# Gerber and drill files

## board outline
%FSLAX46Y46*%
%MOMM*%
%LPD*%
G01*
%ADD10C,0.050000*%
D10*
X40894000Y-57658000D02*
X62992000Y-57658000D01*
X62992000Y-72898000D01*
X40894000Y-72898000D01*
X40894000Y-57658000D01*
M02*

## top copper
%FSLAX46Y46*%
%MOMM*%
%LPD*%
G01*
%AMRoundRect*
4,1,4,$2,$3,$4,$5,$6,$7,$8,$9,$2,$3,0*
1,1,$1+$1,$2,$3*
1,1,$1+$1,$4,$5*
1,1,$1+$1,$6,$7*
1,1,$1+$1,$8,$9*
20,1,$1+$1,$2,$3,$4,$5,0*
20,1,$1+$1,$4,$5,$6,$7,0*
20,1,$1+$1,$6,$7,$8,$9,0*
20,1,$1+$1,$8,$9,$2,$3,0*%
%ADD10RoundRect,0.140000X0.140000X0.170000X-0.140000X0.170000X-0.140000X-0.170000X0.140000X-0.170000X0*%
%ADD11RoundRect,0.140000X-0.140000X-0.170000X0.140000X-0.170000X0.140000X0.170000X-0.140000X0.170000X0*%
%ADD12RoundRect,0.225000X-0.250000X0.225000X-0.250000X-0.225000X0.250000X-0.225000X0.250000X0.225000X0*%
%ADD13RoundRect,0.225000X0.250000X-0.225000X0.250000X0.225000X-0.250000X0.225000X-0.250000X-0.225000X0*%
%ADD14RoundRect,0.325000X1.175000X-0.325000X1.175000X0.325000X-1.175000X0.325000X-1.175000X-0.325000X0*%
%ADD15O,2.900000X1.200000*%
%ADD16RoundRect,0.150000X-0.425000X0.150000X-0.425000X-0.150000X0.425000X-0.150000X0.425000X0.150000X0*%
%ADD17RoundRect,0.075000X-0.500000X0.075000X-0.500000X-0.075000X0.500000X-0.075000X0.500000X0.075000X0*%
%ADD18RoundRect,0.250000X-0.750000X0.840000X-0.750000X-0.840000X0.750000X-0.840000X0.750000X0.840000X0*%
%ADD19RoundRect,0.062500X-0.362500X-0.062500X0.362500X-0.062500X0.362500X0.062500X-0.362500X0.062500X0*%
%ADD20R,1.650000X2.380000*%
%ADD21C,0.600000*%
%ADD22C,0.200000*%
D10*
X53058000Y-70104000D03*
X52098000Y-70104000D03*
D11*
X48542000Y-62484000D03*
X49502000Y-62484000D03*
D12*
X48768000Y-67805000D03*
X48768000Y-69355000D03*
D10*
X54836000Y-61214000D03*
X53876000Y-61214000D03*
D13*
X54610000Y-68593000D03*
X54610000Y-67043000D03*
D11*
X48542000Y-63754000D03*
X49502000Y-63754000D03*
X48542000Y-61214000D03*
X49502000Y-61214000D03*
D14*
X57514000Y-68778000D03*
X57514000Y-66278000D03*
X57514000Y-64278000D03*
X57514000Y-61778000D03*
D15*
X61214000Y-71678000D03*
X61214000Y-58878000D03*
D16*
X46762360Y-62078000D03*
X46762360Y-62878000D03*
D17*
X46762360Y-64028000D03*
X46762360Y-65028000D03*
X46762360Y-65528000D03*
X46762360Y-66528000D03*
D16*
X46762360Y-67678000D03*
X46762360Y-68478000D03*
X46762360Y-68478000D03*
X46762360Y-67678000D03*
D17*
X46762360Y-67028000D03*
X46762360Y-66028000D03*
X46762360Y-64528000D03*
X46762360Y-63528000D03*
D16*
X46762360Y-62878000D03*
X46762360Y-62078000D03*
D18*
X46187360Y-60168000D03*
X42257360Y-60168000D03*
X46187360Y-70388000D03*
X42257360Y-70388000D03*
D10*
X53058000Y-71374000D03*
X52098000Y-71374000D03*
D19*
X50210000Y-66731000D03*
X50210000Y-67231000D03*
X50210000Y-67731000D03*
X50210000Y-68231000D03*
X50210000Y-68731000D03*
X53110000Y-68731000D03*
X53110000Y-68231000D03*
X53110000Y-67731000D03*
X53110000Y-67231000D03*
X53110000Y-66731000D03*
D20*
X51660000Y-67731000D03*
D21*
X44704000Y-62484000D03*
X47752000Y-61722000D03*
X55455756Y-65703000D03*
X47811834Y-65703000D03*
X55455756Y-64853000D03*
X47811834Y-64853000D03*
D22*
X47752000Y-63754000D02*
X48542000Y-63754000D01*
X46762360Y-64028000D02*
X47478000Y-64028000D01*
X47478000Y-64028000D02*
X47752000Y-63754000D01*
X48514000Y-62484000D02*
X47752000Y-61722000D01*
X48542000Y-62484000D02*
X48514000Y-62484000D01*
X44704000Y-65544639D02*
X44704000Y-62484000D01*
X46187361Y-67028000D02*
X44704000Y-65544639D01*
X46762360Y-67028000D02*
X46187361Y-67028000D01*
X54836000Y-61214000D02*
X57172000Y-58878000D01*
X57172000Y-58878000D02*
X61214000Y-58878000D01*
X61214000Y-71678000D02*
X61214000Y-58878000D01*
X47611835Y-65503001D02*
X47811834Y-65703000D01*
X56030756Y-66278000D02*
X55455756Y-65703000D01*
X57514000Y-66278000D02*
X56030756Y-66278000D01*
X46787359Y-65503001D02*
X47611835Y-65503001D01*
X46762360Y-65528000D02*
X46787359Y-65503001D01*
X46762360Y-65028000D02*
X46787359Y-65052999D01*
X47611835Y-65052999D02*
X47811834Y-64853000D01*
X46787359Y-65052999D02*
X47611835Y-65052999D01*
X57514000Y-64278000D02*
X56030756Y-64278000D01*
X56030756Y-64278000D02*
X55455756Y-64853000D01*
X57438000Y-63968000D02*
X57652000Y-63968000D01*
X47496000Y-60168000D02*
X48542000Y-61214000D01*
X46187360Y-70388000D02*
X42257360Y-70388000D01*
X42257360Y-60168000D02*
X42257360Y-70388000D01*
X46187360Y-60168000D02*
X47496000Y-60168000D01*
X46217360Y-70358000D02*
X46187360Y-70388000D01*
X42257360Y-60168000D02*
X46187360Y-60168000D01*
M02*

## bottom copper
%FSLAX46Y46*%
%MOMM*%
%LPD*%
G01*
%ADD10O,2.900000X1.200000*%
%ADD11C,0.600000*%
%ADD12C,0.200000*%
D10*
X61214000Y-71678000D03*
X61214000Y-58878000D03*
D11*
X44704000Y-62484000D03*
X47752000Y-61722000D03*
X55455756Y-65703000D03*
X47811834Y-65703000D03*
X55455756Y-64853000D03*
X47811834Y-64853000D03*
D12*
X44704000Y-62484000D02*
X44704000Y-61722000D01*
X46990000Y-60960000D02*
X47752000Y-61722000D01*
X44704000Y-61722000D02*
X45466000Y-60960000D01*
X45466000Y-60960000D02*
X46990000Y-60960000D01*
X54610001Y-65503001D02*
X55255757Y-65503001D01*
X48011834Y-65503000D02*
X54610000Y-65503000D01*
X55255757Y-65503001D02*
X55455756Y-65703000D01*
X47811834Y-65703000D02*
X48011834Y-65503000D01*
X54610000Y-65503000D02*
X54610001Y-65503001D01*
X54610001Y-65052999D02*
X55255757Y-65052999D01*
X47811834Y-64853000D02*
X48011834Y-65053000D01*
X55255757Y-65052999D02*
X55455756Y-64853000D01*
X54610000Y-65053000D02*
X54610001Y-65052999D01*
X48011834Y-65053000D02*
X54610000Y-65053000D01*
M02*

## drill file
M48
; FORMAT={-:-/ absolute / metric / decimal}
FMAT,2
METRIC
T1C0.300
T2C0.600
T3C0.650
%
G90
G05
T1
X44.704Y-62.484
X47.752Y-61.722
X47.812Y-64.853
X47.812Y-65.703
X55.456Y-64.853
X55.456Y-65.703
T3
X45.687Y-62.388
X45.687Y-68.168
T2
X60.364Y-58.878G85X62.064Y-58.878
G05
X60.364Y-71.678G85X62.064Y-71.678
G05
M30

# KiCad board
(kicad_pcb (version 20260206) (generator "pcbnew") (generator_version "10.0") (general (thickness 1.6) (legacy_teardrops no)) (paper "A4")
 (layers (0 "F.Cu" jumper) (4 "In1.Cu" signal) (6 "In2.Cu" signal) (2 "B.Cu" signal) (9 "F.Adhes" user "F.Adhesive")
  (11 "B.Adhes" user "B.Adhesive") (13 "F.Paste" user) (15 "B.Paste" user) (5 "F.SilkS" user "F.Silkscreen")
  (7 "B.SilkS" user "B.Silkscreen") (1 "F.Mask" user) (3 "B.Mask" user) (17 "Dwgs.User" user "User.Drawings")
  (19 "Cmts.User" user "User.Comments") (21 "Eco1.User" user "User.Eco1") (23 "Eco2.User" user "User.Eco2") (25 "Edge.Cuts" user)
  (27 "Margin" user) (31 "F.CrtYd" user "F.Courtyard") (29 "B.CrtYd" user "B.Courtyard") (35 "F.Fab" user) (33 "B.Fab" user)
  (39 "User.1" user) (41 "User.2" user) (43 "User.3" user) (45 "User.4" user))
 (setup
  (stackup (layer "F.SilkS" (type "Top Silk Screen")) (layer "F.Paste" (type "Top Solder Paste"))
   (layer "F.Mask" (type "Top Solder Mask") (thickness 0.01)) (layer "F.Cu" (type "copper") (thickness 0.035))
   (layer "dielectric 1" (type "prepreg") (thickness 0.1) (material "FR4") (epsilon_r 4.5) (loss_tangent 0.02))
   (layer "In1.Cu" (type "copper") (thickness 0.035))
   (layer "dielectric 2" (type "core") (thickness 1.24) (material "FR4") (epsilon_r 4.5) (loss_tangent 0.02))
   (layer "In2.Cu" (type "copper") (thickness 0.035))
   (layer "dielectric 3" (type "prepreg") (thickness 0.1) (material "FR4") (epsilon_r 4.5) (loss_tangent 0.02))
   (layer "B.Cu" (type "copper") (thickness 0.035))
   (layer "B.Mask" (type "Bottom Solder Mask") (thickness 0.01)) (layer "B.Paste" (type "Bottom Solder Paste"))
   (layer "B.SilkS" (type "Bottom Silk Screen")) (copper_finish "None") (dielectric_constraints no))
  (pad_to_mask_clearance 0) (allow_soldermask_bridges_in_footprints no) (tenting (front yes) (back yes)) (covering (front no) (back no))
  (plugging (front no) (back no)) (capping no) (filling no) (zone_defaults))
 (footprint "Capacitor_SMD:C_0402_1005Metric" (layer "F.Cu") (at 52.578 70.104 180)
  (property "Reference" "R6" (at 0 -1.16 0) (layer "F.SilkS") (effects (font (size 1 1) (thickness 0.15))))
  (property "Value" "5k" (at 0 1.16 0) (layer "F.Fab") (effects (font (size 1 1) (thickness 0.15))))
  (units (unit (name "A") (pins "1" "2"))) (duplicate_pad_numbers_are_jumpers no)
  (pad "1" smd roundrect (at -0.48 0 180) (size 0.56 0.62) (layers "F.Cu" "F.Mask" "F.Paste") (roundrect_rratio 0.25) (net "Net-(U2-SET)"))
  (pad "2" smd roundrect (at 0.48 0 180) (size 0.56 0.62) (layers "F.Cu" "F.Mask" "F.Paste") (roundrect_rratio 0.25) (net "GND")))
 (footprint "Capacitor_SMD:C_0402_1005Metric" (layer "F.Cu") (at 49.022 62.484)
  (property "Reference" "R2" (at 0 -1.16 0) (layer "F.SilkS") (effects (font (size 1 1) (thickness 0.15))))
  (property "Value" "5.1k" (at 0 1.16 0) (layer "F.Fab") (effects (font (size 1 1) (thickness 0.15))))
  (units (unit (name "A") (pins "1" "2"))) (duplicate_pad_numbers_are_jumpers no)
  (pad "1" smd roundrect (at -0.48 0) (size 0.56 0.62) (layers "F.Cu" "F.Mask" "F.Paste") (roundrect_rratio 0.25) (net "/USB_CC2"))
  (pad "2" smd roundrect (at 0.48 0) (size 0.56 0.62) (layers "F.Cu" "F.Mask" "F.Paste") (roundrect_rratio 0.25) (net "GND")))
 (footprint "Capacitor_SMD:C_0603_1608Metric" (layer "F.Cu") (at 48.768 68.58 -90)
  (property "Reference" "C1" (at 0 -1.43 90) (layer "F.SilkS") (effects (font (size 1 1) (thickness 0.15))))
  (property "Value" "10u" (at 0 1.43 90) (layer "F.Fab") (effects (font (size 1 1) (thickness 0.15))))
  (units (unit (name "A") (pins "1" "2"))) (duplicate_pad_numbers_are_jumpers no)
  (pad "1" smd roundrect (at -0.775 0 270) (size 0.9 0.95) (layers "F.Cu" "F.Mask" "F.Paste") (roundrect_rratio 0.25) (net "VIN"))
  (pad "2" smd roundrect (at 0.775 0 270) (size 0.9 0.95) (layers "F.Cu" "F.Mask" "F.Paste") (roundrect_rratio 0.25) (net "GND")))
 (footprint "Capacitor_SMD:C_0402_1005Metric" (layer "F.Cu") (at 54.356 61.214 180)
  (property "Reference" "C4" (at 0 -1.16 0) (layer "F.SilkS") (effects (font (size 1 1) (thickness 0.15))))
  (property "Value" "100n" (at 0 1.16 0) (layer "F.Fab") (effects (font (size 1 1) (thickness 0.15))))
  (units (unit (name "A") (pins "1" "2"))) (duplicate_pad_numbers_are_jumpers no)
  (pad "1" smd roundrect (at -0.48 0 180) (size 0.56 0.62) (layers "F.Cu" "F.Mask" "F.Paste") (roundrect_rratio 0.25)
   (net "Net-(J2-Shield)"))
  (pad "2" smd roundrect (at 0.48 0 180) (size 0.56 0.62) (layers "F.Cu" "F.Mask" "F.Paste") (roundrect_rratio 0.25) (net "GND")))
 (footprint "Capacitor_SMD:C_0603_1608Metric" (layer "F.Cu") (at 54.61 67.818 90)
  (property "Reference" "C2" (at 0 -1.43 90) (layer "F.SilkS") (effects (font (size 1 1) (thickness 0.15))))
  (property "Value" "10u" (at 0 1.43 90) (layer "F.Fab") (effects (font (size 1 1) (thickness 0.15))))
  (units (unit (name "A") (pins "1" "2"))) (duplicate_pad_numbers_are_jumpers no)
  (pad "1" smd roundrect (at -0.775 0 90) (size 0.9 0.95) (layers "F.Cu" "F.Mask" "F.Paste") (roundrect_rratio 0.25) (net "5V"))
  (pad "2" smd roundrect (at 0.775 0 90) (size 0.9 0.95) (layers "F.Cu" "F.Mask" "F.Paste") (roundrect_rratio 0.25) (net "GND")))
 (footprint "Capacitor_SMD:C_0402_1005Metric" (layer "F.Cu") (at 49.022 63.754)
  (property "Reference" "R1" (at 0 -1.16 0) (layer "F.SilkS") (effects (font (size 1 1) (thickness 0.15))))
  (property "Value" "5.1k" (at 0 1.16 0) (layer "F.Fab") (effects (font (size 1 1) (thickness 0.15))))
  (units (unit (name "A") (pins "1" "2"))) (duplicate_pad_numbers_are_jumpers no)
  (pad "1" smd roundrect (at -0.48 0) (size 0.56 0.62) (layers "F.Cu" "F.Mask" "F.Paste") (roundrect_rratio 0.25) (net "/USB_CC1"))
  (pad "2" smd roundrect (at 0.48 0) (size 0.56 0.62) (layers "F.Cu" "F.Mask" "F.Paste") (roundrect_rratio 0.25) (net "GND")))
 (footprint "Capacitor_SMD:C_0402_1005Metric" (layer "F.Cu") (at 49.022 61.214)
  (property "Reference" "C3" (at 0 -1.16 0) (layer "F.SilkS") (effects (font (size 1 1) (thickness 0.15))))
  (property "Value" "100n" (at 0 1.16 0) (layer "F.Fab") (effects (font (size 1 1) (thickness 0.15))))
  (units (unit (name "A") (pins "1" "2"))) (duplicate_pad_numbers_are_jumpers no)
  (pad "1" smd roundrect (at -0.48 0) (size 0.56 0.62) (layers "F.Cu" "F.Mask" "F.Paste") (roundrect_rratio 0.25) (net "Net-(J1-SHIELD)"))
  (pad "2" smd roundrect (at 0.48 0) (size 0.56 0.62) (layers "F.Cu" "F.Mask" "F.Paste") (roundrect_rratio 0.25) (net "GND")))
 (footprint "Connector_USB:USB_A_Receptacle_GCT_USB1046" (layer "F.Cu") (at 64.764 65.278 90)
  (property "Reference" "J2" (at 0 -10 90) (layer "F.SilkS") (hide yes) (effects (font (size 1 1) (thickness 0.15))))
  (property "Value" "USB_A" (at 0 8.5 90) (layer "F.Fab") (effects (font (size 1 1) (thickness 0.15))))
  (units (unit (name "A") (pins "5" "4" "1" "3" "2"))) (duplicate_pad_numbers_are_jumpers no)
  (pad "" smd oval (at -6.4 -3.55 90) (size 1.2 2.9) (layers "F.Paste") (thermal_bridge_angle 45))
  (pad "" smd oval (at 6.4 -3.55 90) (size 1.2 2.9) (layers "F.Paste") (thermal_bridge_angle 45))
  (pad "1" smd roundrect (at -3.5 -7.25 90) (size 1.3 3) (layers "F.Cu" "F.Mask" "F.Paste") (roundrect_rratio 0.25) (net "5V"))
  (pad "2" smd roundrect (at -1 -7.25 90) (size 1.3 3) (layers "F.Cu" "F.Mask" "F.Paste") (roundrect_rratio 0.25) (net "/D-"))
  (pad "3" smd roundrect (at 1 -7.25 90) (size 1.3 3) (layers "F.Cu" "F.Mask" "F.Paste") (roundrect_rratio 0.25) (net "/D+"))
  (pad "4" smd roundrect (at 3.5 -7.25 90) (size 1.3 3) (layers "F.Cu" "F.Mask" "F.Paste") (roundrect_rratio 0.25) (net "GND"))
  (pad "SH" thru_hole oval (at -6.4 -3.55 90) (size 1.2 2.9) (drill oval 0.6 2.3) (layers "*.Cu" "*.Mask") (remove_unused_layers no)
   (thermal_bridge_angle 45))
  (pad "SH" thru_hole oval (at 6.4 -3.55 90) (size 1.2 2.9) (drill oval 0.6 2.3) (layers "*.Cu" "*.Mask") (remove_unused_layers no)
   (thermal_bridge_angle 45)))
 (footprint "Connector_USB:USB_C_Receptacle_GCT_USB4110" (layer "F.Cu") (at 43.08236 65.278 -90)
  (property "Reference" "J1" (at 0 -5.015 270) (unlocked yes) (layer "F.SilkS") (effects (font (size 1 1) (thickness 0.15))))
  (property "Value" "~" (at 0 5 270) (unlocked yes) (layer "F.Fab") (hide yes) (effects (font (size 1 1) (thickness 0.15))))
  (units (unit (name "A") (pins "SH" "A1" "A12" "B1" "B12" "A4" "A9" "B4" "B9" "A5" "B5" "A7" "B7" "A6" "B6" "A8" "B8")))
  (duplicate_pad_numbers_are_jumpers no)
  (pad "" np_thru_hole circle (at -2.89 -2.605 270) (size 0.65 0.65) (drill 0.65) (layers "*.Cu" "*.Mask"))
  (pad "" np_thru_hole circle (at 2.89 -2.605 270) (size 0.65 0.65) (drill 0.65) (layers "*.Cu" "*.Mask"))
  (pad "A1" smd roundrect (at -3.2 -3.68 270) (size 0.6 1.15) (layers "F.Cu" "F.Mask" "F.Paste") (roundrect_rratio 0.25) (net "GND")
   (thermal_bridge_angle 45))
  (pad "A4" smd roundrect (at -2.4 -3.68 270) (size 0.6 1.15) (layers "F.Cu" "F.Mask" "F.Paste") (roundrect_rratio 0.25) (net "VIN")
   (thermal_bridge_angle 45))
  (pad "A5" smd roundrect (at -1.25 -3.68 270) (size 0.3 1.15) (layers "F.Cu" "F.Mask" "F.Paste") (roundrect_rratio 0.25) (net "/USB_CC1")
   (thermal_bridge_angle 45))
  (pad "A6" smd roundrect (at -0.25 -3.68 270) (size 0.3 1.15) (layers "F.Cu" "F.Mask" "F.Paste") (roundrect_rratio 0.25) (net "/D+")
   (thermal_bridge_angle 45))
  (pad "A7" smd roundrect (at 0.25 -3.68 270) (size 0.3 1.15) (layers "F.Cu" "F.Mask" "F.Paste") (roundrect_rratio 0.25) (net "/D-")
   (thermal_bridge_angle 45))
  (pad "A8" smd roundrect (at 1.25 -3.68 270) (size 0.3 1.15) (layers "F.Cu" "F.Mask" "F.Paste") (roundrect_rratio 0.25)
   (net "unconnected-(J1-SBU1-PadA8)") (thermal_bridge_angle 45))
  (pad "A9" smd roundrect (at 2.4 -3.68 270) (size 0.6 1.15) (layers "F.Cu" "F.Mask" "F.Paste") (roundrect_rratio 0.25) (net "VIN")
   (thermal_bridge_angle 45))
  (pad "A12" smd roundrect (at 3.2 -3.68 270) (size 0.6 1.15) (layers "F.Cu" "F.Mask" "F.Paste") (roundrect_rratio 0.25) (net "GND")
   (thermal_bridge_angle 45))
  (pad "B1" smd roundrect (at 3.2 -3.68 270) (size 0.6 1.15) (layers "F.Cu" "F.Mask" "F.Paste") (roundrect_rratio 0.25) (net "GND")
   (thermal_bridge_angle 45))
  (pad "B4" smd roundrect (at 2.4 -3.68 270) (size 0.6 1.15) (layers "F.Cu" "F.Mask" "F.Paste") (roundrect_rratio 0.25) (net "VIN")
   (thermal_bridge_angle 45))
  (pad "B5" smd roundrect (at 1.75 -3.68 270) (size 0.3 1.15) (layers "F.Cu" "F.Mask" "F.Paste") (roundrect_rratio 0.25) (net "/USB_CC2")
   (thermal_bridge_angle 45))
  (pad "B6" smd roundrect (at 0.75 -3.68 270) (size 0.3 1.15) (layers "F.Cu" "F.Mask" "F.Paste") (roundrect_rratio 0.25) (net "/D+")
   (thermal_bridge_angle 45))
  (pad "B7" smd roundrect (at -0.75 -3.68 270) (size 0.3 1.15) (layers "F.Cu" "F.Mask" "F.Paste") (roundrect_rratio 0.25) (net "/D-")
   (thermal_bridge_angle 45))
  (pad "B8" smd roundrect (at -1.75 -3.68 270) (size 0.3 1.15) (layers "F.Cu" "F.Mask" "F.Paste") (roundrect_rratio 0.25)
   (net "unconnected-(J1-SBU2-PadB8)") (thermal_bridge_angle 45))
  (pad "B9" smd roundrect (at -2.4 -3.68 270) (size 0.6 1.15) (layers "F.Cu" "F.Mask" "F.Paste") (roundrect_rratio 0.25) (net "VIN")
   (thermal_bridge_angle 45))
  (pad "B12" smd roundrect (at -3.2 -3.68 270) (size 0.6 1.15) (layers "F.Cu" "F.Mask" "F.Paste") (roundrect_rratio 0.25) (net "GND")
   (thermal_bridge_angle 45))
  (pad "SH" smd roundrect (at -5.11 -3.105 270) (size 2.18 2) (layers "F.Cu" "F.Mask" "F.Paste") (roundrect_rratio 0.125)
   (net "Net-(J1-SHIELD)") (thermal_bridge_angle 45))
  (pad "SH" smd roundrect (at -5.11 0.825 270) (size 2.18 2) (layers "F.Cu" "F.Mask" "F.Paste") (roundrect_rratio 0.125)
   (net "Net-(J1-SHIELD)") (thermal_bridge_angle 45))
  (pad "SH" smd roundrect (at 5.11 -3.105 270) (size 2.18 2) (layers "F.Cu" "F.Mask" "F.Paste") (roundrect_rratio 0.125)
   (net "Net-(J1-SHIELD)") (thermal_bridge_angle 45))
  (pad "SH" smd roundrect (at 5.11 0.825 270) (size 2.18 2) (layers "F.Cu" "F.Mask" "F.Paste") (roundrect_rratio 0.125)
   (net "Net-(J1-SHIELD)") (thermal_bridge_angle 45)))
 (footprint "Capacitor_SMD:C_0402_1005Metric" (layer "F.Cu") (at 52.578 71.374 180)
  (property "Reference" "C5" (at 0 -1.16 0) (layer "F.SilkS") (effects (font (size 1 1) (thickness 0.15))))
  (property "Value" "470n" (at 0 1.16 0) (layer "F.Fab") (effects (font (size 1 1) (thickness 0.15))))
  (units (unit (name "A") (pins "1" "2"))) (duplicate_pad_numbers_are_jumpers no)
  (pad "1" smd roundrect (at -0.48 0 180) (size 0.56 0.62) (layers "F.Cu" "F.Mask" "F.Paste") (roundrect_rratio 0.25) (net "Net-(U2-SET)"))
  (pad "2" smd roundrect (at 0.48 0 180) (size 0.56 0.62) (layers "F.Cu" "F.Mask" "F.Paste") (roundrect_rratio 0.25) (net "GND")))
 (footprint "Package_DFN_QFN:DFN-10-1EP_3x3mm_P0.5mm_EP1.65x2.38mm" (layer "F.Cu") (at 51.66 67.731)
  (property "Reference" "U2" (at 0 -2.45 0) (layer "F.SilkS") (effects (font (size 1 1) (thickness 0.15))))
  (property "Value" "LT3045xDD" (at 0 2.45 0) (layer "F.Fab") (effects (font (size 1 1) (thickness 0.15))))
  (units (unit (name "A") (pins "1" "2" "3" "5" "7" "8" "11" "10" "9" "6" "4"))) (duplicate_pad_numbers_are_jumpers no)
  (pad "" smd roundrect (at -0.41 -0.595) (size 0.67 0.96) (layers "F.Paste") (roundrect_rratio 0.25))
  (pad "" smd roundrect (at -0.41 0.595) (size 0.67 0.96) (layers "F.Paste") (roundrect_rratio 0.25))
  (pad "" smd roundrect (at 0.41 -0.595) (size 0.67 0.96) (layers "F.Paste") (roundrect_rratio 0.25))
  (pad "" smd roundrect (at 0.41 0.595) (size 0.67 0.96) (layers "F.Paste") (roundrect_rratio 0.25))
  (pad "1" smd roundrect (at -1.45 -1) (size 0.85 0.25) (layers "F.Cu" "F.Mask" "F.Paste") (roundrect_rratio 0.25) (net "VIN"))
  (pad "2" smd roundrect (at -1.45 -0.5) (size 0.85 0.25) (layers "F.Cu" "F.Mask" "F.Paste") (roundrect_rratio 0.25) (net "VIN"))
  (pad "3" smd roundrect (at -1.45 0) (size 0.85 0.25) (layers "F.Cu" "F.Mask" "F.Paste") (roundrect_rratio 0.25) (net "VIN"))
  (pad "4" smd roundrect (at -1.45 0.5) (size 0.85 0.25) (layers "F.Cu" "F.Mask" "F.Paste") (roundrect_rratio 0.25)
   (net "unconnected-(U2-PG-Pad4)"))
  (pad "5" smd roundrect (at -1.45 1) (size 0.85 0.25) (layers "F.Cu" "F.Mask" "F.Paste") (roundrect_rratio 0.25) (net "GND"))
  (pad "6" smd roundrect (at 1.45 1) (size 0.85 0.25) (layers "F.Cu" "F.Mask" "F.Paste") (roundrect_rratio 0.25) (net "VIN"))
  (pad "7" smd roundrect (at 1.45 0.5) (size 0.85 0.25) (layers "F.Cu" "F.Mask" "F.Paste") (roundrect_rratio 0.25) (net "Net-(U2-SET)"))
  (pad "8" smd roundrect (at 1.45 0) (size 0.85 0.25) (layers "F.Cu" "F.Mask" "F.Paste") (roundrect_rratio 0.25) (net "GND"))
  (pad "9" smd roundrect (at 1.45 -0.5) (size 0.85 0.25) (layers "F.Cu" "F.Mask" "F.Paste") (roundrect_rratio 0.25) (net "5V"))
  (pad "10" smd roundrect (at 1.45 -1) (size 0.85 0.25) (layers "F.Cu" "F.Mask" "F.Paste") (roundrect_rratio 0.25) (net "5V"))
  (pad "11" smd rect (at 0 0) (size 1.65 2.38) (layers "F.Cu" "F.Mask") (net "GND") (zone_connect 2)))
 (gr_rect (start 40.894 57.658) (end 62.992 72.898) (stroke (width 0.05) (type default)) (fill no) (layer "Edge.Cuts"))
 (segment (start 47.752 63.754) (end 48.542 63.754) (width 0.2) (layer "F.Cu") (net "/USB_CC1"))
 (segment (start 46.76236 64.028) (end 47.478 64.028) (width 0.2) (layer "F.Cu") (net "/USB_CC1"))
 (segment (start 47.478 64.028) (end 47.752 63.754) (width 0.2) (layer "F.Cu") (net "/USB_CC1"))
 (segment (start 48.514 62.484) (end 47.752 61.722) (width 0.2) (layer "F.Cu") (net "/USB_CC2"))
 (segment (start 48.542 62.484) (end 48.514 62.484) (width 0.2) (layer "F.Cu") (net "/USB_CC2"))
 (segment (start 44.704 65.544639) (end 44.704 62.484) (width 0.2) (layer "F.Cu") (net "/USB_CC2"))
 (segment (start 46.187361 67.028) (end 44.704 65.544639) (width 0.2) (layer "F.Cu") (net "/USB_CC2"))
 (segment (start 46.76236 67.028) (end 46.187361 67.028) (width 0.2) (layer "F.Cu") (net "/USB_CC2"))
 (via (at 44.704 62.484) (size 0.6) (drill 0.3) (layers "F.Cu" "B.Cu") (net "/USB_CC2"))
 (via (at 47.752 61.722) (size 0.6) (drill 0.3) (layers "F.Cu" "B.Cu") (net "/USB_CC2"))
 (segment (start 44.704 62.484) (end 44.704 61.722) (width 0.2) (layer "B.Cu") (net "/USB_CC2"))
 (segment (start 46.99 60.96) (end 47.752 61.722) (width 0.2) (layer "B.Cu") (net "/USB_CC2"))
 (segment (start 44.704 61.722) (end 45.466 60.96) (width 0.2) (layer "B.Cu") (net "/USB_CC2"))
 (segment (start 45.466 60.96) (end 46.99 60.96) (width 0.2) (layer "B.Cu") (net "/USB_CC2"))
 (segment (start 54.836 61.214) (end 57.172 58.878) (width 0.2) (layer "F.Cu") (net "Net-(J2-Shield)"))
 (segment (start 57.172 58.878) (end 61.214 58.878) (width 0.2) (layer "F.Cu") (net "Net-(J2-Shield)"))
 (segment (start 61.214 71.678) (end 61.214 58.878) (width 0.2) (layer "F.Cu") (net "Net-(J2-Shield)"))
 (segment (start 47.611835 65.503001) (end 47.811834 65.703) (width 0.2) (layer "F.Cu") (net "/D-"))
 (segment (start 56.030756 66.278) (end 55.455756 65.703) (width 0.2) (layer "F.Cu") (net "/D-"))
 (segment (start 57.514 66.278) (end 56.030756 66.278) (width 0.2) (layer "F.Cu") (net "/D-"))
 (segment (start 46.787359 65.503001) (end 47.611835 65.503001) (width 0.2) (layer "F.Cu") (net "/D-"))
 (segment (start 46.76236 65.528) (end 46.787359 65.503001) (width 0.2) (layer "F.Cu") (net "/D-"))
 (via (at 55.455756 65.703) (size 0.6) (drill 0.3) (layers "F.Cu" "B.Cu") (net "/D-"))
 (via (at 47.811834 65.703) (size 0.6) (drill 0.3) (layers "F.Cu" "B.Cu") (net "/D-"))
 (segment (start 54.610001 65.503001) (end 55.255757 65.503001) (width 0.2) (layer "B.Cu") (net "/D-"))
 (segment (start 48.011834 65.503) (end 54.61 65.503) (width 0.2) (layer "B.Cu") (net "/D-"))
 (segment (start 55.255757 65.503001) (end 55.455756 65.703) (width 0.2) (layer "B.Cu") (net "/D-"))
 (segment (start 47.811834 65.703) (end 48.011834 65.503) (width 0.2) (layer "B.Cu") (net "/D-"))
 (segment (start 54.61 65.503) (end 54.610001 65.503001) (width 0.2) (layer "B.Cu") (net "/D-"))
 (segment (start 46.76236 65.028) (end 46.787359 65.052999) (width 0.2) (layer "F.Cu") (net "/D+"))
 (segment (start 47.611835 65.052999) (end 47.811834 64.853) (width 0.2) (layer "F.Cu") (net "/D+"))
 (segment (start 46.787359 65.052999) (end 47.611835 65.052999) (width 0.2) (layer "F.Cu") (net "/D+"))
 (segment (start 57.514 64.278) (end 56.030756 64.278) (width 0.2) (layer "F.Cu") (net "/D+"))
 (segment (start 56.030756 64.278) (end 55.455756 64.853) (width 0.2) (layer "F.Cu") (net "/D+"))
 (segment (start 57.438 63.968) (end 57.652 63.968) (width 0.2) (layer "F.Cu") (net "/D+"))
 (via (at 55.455756 64.853) (size 0.6) (drill 0.3) (layers "F.Cu" "B.Cu") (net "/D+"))
 (via (at 47.811834 64.853) (size 0.6) (drill 0.3) (layers "F.Cu" "B.Cu") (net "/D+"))
 (segment (start 54.610001 65.052999) (end 55.255757 65.052999) (width 0.2) (layer "B.Cu") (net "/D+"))
 (segment (start 47.811834 64.853) (end 48.011834 65.053) (width 0.2) (layer "B.Cu") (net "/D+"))
 (segment (start 55.255757 65.052999) (end 55.455756 64.853) (width 0.2) (layer "B.Cu") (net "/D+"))
 (segment (start 54.61 65.053) (end 54.610001 65.052999) (width 0.2) (layer "B.Cu") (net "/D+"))
 (segment (start 48.011834 65.053) (end 54.61 65.053) (width 0.2) (layer "B.Cu") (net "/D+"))
 (segment (start 47.496 60.168) (end 48.542 61.214) (width 0.2) (layer "F.Cu") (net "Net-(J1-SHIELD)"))
 (segment (start 46.18736 70.388) (end 42.25736 70.388) (width 0.2) (layer "F.Cu") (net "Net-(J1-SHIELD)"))
 (segment (start 42.25736 60.168) (end 42.25736 70.388) (width 0.2) (layer "F.Cu") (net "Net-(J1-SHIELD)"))
 (segment (start 46.18736 60.168) (end 47.496 60.168) (width 0.2) (layer "F.Cu") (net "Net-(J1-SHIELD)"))
 (segment (start 46.21736 70.358) (end 46.18736 70.388) (width 0.2) (layer "F.Cu") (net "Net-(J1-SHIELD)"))
 (segment (start 42.25736 60.168) (end 46.18736 60.168) (width 0.2) (layer "F.Cu") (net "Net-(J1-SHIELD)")))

